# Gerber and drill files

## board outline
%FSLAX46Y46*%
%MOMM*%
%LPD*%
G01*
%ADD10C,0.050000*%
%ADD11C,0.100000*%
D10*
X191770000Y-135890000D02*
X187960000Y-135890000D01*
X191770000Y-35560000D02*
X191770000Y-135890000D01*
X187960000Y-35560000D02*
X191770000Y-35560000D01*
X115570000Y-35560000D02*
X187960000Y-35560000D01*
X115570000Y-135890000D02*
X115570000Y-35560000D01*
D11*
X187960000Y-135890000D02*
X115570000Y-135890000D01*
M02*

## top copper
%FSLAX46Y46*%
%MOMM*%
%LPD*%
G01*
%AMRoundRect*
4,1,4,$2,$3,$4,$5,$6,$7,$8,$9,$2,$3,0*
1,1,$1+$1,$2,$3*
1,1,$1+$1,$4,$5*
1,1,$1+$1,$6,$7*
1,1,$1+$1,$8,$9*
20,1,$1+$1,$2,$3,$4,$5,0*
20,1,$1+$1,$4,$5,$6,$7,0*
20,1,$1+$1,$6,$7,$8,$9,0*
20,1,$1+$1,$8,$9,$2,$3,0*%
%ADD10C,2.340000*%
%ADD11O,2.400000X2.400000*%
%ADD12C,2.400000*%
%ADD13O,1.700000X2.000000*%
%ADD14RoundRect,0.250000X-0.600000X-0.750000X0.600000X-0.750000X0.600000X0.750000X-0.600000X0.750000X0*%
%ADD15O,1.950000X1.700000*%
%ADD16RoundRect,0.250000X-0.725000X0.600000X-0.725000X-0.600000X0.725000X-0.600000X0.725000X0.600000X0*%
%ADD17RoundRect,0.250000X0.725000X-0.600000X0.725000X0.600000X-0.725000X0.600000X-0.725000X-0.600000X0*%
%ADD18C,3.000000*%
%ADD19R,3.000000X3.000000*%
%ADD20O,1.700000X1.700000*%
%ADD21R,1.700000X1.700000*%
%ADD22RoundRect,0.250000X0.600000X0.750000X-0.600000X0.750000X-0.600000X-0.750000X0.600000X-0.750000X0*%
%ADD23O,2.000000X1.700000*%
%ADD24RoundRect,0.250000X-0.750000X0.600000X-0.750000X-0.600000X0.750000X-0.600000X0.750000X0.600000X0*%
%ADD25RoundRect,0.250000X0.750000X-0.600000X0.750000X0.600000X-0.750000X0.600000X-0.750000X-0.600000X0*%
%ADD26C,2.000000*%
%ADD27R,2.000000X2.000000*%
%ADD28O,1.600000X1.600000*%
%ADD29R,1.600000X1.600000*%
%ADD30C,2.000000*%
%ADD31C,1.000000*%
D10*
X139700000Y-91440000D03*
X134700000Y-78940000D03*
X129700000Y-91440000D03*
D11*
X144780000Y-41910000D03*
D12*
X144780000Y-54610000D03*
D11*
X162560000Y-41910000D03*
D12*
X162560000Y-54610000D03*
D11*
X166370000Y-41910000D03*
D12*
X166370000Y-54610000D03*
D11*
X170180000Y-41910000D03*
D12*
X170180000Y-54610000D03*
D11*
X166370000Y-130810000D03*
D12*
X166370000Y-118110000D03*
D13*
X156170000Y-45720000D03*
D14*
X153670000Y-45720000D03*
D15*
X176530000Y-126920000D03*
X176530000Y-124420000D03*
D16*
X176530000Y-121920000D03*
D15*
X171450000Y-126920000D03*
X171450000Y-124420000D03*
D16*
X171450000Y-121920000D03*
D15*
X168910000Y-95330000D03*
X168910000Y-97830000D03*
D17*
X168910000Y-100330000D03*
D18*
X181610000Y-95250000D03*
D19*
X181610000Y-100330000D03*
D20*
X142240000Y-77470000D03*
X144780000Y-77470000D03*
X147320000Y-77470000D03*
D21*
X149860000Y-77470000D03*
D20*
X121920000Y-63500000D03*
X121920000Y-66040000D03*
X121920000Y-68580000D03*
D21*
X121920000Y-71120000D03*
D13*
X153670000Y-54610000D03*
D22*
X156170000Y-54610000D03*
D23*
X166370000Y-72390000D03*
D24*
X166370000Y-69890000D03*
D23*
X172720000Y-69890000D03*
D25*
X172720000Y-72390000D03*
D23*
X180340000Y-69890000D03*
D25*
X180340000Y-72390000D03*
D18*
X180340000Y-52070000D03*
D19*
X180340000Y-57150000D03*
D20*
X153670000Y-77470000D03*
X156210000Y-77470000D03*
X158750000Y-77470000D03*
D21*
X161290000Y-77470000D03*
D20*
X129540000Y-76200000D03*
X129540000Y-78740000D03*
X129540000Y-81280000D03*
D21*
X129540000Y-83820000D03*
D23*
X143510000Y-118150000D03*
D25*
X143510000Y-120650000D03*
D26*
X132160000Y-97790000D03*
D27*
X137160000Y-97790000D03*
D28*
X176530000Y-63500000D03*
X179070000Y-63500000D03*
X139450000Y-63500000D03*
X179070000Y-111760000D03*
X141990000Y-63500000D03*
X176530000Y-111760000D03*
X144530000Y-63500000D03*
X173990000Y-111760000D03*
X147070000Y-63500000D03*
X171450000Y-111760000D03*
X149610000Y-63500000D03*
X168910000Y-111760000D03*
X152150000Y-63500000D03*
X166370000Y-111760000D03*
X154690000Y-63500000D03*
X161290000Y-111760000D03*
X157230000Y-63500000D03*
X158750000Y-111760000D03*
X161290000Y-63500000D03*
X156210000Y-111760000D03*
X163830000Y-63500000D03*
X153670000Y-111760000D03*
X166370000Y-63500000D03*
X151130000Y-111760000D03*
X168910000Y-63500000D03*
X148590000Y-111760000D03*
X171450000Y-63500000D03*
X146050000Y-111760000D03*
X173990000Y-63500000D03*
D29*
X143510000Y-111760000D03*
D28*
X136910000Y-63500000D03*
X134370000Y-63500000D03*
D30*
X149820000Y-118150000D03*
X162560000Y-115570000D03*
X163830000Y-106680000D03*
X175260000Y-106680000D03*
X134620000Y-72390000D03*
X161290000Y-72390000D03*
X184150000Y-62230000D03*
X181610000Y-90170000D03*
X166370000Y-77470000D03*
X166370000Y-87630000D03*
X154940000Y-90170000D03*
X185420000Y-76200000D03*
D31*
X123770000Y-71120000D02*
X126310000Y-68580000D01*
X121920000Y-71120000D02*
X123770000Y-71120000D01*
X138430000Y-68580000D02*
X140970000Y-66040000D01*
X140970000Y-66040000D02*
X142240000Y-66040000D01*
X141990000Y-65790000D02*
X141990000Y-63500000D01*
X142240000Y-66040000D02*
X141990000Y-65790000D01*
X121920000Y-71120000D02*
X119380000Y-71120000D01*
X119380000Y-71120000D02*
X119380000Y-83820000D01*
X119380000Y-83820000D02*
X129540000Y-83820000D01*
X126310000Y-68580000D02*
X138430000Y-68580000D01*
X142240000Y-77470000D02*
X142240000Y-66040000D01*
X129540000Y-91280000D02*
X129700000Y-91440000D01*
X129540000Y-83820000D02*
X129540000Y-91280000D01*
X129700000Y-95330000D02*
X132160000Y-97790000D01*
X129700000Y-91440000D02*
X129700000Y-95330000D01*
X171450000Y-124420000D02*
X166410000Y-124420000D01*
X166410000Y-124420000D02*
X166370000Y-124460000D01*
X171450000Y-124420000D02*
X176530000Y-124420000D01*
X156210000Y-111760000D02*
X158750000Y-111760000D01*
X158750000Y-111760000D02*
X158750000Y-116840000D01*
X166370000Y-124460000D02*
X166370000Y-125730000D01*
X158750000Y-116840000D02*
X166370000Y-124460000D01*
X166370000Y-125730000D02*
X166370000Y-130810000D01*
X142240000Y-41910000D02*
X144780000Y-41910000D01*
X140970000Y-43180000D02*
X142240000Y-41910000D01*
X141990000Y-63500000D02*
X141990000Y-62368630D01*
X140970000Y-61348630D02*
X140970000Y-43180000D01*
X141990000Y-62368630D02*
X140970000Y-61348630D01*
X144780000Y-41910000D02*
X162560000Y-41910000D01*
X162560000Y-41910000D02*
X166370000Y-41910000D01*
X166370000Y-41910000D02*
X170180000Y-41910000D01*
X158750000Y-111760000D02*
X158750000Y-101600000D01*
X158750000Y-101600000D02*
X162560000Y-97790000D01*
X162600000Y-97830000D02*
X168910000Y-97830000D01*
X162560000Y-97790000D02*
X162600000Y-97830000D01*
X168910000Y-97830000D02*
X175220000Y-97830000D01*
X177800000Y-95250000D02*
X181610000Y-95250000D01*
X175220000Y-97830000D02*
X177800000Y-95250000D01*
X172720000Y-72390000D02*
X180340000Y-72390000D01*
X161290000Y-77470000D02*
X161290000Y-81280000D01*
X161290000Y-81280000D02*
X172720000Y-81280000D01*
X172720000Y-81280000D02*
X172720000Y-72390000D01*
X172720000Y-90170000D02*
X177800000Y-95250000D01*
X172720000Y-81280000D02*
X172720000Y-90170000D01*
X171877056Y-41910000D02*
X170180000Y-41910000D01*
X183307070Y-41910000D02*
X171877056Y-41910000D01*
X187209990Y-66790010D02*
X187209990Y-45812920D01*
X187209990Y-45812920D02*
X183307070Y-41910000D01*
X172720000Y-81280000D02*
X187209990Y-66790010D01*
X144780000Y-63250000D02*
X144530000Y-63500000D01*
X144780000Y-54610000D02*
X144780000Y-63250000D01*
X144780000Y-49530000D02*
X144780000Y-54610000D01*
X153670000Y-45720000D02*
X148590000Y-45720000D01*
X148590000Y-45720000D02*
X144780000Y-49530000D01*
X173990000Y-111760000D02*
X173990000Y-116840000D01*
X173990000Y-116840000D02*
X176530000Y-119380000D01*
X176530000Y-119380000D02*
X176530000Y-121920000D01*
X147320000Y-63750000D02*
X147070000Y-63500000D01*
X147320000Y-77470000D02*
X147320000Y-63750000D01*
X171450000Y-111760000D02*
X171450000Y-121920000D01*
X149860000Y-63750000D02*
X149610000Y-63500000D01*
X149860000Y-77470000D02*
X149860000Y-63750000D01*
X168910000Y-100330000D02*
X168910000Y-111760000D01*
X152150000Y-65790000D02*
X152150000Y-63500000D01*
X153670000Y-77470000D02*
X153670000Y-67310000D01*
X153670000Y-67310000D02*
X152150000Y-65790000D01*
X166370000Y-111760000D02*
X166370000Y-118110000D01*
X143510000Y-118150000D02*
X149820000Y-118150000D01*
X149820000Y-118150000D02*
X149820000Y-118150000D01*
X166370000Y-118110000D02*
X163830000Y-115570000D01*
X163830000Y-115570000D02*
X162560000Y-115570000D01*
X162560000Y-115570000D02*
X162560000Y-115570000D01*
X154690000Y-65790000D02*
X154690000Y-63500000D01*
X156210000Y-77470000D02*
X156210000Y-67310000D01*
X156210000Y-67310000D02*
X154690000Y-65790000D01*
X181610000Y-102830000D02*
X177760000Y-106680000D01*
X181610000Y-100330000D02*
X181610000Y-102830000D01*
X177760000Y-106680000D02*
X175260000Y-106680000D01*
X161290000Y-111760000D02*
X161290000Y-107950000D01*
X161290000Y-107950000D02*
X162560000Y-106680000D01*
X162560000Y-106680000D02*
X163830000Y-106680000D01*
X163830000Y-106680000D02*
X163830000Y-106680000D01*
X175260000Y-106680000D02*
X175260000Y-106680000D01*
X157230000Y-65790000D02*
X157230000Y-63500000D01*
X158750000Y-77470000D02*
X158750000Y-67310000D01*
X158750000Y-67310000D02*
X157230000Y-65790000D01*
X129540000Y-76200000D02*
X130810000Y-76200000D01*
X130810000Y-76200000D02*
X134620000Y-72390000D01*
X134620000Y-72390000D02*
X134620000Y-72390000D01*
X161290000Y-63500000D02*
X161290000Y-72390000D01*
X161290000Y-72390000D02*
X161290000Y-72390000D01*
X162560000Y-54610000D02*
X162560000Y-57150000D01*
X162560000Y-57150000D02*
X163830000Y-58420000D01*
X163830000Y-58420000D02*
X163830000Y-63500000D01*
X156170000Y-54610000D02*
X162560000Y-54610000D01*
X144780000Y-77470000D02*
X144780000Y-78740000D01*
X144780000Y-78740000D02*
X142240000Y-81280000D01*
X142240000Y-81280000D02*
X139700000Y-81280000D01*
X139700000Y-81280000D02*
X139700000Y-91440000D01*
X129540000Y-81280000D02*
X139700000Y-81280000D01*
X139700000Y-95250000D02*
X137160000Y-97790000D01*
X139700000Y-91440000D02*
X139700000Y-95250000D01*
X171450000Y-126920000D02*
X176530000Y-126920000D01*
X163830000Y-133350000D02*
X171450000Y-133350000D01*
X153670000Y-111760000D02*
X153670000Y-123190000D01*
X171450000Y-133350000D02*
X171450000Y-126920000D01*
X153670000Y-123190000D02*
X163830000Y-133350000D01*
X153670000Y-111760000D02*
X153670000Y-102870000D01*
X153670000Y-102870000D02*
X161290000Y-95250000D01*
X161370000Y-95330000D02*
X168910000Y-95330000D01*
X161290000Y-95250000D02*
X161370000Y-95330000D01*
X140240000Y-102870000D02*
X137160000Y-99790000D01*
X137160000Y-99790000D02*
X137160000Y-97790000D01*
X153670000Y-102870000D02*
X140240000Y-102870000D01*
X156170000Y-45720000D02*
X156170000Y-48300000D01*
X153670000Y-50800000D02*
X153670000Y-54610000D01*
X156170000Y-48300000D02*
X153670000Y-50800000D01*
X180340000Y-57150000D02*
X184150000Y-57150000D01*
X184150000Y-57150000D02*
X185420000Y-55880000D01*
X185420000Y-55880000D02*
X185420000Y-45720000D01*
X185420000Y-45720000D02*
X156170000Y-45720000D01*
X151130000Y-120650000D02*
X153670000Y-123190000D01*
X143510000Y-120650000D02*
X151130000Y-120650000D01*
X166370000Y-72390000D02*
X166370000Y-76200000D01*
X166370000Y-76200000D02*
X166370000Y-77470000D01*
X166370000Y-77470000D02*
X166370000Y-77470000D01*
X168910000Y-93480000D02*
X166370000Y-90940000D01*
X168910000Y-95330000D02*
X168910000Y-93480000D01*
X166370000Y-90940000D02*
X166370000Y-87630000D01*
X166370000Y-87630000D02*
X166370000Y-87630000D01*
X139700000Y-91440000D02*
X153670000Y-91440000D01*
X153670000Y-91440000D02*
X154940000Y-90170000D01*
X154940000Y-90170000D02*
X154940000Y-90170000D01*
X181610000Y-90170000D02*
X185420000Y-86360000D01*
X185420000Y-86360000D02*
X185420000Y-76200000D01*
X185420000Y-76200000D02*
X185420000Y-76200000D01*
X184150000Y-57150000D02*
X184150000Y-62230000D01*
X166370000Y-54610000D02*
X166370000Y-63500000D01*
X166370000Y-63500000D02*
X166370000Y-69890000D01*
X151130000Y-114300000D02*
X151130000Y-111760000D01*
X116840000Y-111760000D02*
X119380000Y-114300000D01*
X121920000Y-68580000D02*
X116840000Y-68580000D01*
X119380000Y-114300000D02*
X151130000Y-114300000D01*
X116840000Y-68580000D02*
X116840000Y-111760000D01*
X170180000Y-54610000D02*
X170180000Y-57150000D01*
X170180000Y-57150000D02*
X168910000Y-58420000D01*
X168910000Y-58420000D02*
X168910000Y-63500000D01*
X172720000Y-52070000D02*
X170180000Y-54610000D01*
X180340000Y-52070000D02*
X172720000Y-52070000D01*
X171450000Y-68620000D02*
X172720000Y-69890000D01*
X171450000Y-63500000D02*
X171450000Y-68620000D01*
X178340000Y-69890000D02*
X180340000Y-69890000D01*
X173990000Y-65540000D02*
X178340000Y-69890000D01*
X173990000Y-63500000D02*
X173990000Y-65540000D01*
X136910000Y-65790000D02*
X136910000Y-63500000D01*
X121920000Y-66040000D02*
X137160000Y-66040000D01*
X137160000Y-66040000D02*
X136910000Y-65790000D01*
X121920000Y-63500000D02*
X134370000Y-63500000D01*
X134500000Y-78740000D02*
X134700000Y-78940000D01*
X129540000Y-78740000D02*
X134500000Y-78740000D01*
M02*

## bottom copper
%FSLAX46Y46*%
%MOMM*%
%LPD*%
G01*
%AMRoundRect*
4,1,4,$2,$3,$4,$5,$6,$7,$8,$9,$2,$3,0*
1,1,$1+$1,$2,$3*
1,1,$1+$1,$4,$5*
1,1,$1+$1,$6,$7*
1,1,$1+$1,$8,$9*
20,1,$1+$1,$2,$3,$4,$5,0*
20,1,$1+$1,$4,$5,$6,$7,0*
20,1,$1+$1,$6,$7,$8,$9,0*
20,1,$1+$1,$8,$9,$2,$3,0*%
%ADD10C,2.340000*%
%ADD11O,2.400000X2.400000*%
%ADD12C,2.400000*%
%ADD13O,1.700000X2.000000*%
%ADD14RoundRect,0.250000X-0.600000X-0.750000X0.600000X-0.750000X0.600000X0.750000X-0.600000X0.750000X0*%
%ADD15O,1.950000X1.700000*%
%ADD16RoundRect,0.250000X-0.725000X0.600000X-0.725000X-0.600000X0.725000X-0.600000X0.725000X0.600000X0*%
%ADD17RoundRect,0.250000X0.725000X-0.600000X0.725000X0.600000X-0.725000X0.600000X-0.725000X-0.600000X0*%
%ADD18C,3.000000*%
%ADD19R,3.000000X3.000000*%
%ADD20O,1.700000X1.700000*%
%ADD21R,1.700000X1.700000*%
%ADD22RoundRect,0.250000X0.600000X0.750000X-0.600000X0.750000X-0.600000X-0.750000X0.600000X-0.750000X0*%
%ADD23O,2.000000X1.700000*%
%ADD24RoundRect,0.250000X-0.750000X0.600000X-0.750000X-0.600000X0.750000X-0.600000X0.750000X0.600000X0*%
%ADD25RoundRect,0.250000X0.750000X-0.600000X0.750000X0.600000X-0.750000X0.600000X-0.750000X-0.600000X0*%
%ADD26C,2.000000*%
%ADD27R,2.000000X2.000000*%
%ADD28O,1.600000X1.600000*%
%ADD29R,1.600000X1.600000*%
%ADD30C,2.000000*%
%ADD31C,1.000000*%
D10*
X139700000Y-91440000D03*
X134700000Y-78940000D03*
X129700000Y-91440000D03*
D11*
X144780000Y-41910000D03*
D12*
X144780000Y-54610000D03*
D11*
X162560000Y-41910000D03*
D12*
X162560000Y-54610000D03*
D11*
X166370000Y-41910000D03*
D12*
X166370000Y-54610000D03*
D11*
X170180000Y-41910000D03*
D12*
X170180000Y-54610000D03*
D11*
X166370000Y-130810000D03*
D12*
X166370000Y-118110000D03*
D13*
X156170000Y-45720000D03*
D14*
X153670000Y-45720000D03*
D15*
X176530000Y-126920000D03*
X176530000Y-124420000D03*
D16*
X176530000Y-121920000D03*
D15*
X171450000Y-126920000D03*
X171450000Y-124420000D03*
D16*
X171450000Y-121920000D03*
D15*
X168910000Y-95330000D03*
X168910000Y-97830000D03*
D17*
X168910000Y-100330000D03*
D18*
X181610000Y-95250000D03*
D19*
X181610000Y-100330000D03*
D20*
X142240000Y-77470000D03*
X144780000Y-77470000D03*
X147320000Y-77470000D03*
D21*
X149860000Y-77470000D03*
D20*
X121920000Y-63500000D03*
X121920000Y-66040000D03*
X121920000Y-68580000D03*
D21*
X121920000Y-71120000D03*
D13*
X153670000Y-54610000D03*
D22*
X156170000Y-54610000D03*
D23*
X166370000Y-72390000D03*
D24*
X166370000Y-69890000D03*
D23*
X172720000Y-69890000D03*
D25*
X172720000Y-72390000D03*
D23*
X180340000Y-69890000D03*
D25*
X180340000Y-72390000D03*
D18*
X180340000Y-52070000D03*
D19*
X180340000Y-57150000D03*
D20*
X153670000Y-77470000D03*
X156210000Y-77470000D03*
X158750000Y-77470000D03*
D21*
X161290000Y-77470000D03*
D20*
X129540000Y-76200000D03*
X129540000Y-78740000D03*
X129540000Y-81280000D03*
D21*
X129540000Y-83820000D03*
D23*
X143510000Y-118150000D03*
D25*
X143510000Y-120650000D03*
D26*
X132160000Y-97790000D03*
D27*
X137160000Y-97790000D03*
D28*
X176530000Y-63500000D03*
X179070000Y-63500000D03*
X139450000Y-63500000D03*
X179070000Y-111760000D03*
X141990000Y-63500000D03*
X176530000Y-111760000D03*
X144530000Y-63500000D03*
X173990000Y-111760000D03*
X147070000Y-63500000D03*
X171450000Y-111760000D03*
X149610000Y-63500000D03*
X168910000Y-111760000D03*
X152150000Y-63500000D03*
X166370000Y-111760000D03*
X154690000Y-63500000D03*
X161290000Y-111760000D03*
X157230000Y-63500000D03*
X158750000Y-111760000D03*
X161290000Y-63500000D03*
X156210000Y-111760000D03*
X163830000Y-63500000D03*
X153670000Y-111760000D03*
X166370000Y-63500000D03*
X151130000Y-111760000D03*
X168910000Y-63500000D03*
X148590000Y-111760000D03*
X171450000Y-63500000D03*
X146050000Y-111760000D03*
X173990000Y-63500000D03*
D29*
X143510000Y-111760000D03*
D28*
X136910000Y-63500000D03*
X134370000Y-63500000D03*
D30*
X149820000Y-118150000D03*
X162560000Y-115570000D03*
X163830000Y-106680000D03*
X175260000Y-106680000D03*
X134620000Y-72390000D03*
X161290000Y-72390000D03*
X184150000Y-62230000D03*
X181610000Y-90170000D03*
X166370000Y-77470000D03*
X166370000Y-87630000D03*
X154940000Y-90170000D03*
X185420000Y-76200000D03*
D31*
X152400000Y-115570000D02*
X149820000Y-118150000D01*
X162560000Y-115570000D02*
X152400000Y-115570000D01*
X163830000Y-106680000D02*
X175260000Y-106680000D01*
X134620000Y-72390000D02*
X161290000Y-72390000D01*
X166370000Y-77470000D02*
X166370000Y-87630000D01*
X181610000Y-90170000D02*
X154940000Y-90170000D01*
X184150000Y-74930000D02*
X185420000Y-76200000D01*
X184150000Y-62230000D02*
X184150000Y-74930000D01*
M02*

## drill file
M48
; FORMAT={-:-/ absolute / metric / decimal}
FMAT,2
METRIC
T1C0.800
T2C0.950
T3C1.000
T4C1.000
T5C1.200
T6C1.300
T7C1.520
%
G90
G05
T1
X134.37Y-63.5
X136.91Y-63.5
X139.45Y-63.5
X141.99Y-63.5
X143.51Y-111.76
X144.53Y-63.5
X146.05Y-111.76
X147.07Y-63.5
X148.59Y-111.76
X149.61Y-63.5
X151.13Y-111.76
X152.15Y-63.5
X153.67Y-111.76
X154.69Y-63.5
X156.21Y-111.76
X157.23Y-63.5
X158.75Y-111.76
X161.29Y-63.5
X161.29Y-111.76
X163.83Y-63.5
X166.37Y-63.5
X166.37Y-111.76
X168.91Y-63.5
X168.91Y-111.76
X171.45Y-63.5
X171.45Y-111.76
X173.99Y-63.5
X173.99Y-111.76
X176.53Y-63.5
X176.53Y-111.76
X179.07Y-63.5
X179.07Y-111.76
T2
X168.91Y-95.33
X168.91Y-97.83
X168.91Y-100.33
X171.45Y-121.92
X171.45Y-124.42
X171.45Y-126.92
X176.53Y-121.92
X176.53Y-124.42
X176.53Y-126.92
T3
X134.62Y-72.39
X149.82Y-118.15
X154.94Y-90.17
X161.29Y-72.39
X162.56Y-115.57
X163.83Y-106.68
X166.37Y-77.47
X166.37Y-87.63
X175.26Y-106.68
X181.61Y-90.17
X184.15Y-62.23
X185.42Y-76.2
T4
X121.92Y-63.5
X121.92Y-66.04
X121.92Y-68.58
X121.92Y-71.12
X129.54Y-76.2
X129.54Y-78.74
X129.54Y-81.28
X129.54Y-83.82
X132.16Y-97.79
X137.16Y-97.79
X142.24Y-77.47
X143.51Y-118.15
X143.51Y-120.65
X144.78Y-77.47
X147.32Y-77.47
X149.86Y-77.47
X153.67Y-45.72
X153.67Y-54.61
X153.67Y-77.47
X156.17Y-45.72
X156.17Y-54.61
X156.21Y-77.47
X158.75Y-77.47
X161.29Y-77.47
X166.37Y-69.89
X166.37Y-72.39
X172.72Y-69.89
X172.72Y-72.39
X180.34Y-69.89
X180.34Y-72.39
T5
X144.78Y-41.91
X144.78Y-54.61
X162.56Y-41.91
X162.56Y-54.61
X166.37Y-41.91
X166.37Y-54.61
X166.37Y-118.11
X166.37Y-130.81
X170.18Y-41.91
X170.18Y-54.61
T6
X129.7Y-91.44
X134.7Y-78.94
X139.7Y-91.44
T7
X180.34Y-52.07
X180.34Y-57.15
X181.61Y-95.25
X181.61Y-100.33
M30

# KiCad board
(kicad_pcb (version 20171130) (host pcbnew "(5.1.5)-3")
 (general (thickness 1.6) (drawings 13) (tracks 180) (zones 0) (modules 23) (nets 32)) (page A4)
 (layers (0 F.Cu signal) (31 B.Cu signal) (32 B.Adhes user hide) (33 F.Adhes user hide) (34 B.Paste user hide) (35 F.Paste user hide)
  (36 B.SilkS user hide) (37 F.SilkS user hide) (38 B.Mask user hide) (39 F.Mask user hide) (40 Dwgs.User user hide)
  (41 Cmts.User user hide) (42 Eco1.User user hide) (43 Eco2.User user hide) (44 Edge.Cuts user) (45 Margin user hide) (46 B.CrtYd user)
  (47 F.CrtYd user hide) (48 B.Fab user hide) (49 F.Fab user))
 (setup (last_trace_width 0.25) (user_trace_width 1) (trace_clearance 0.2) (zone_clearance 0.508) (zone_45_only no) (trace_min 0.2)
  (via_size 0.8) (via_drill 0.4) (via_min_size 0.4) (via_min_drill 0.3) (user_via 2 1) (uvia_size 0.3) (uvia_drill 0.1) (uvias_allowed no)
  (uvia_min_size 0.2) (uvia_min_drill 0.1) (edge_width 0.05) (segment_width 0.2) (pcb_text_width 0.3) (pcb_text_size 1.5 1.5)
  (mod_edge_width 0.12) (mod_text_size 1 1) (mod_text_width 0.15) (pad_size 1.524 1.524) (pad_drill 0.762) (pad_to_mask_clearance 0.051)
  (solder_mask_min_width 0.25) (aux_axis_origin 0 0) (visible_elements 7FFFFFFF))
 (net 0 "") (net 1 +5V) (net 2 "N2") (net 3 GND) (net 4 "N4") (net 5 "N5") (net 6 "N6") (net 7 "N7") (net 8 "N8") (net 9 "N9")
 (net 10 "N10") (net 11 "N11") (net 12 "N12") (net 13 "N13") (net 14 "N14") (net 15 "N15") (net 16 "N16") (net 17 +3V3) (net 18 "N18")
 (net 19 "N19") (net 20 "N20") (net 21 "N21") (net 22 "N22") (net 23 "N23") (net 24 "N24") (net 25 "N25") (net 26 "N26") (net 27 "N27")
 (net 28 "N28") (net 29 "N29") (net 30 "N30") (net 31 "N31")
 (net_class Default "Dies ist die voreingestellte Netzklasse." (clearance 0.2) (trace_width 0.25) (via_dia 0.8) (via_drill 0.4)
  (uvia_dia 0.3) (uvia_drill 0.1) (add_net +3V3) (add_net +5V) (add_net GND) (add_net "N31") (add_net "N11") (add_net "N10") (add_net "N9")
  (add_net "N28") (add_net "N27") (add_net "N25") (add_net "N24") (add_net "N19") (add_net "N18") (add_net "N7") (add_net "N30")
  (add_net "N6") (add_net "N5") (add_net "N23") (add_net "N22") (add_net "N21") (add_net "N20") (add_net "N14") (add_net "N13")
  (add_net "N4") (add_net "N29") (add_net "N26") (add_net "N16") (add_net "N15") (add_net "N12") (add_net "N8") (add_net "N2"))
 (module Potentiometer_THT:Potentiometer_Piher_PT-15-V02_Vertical (layer F.Cu) (at 139.7 91.44 90)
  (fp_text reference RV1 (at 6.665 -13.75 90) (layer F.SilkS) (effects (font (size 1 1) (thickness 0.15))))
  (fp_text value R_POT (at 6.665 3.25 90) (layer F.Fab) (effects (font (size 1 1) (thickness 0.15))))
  (pad 1 thru_hole circle (at 0 0 90) (size 2.34 2.34) (drill 1.3) (layers *.Cu *.Mask) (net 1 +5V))
  (pad 2 thru_hole circle (at 12.5 -5 90) (size 2.34 2.34) (drill 1.3) (layers *.Cu *.Mask) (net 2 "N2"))
  (pad 3 thru_hole circle (at 0 -10 90) (size 2.34 2.34) (drill 1.3) (layers *.Cu *.Mask) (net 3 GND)))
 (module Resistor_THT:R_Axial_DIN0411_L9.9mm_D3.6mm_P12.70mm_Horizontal (layer F.Cu) (at 144.78 54.61 90)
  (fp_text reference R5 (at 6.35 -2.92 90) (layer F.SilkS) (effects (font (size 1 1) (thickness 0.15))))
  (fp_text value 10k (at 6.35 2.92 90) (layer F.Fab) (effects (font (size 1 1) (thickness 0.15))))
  (pad 2 thru_hole oval (at 12.7 0 90) (size 2.4 2.4) (drill 1.2) (layers *.Cu *.Mask) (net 3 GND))
  (pad 1 thru_hole circle (at 0 0 90) (size 2.4 2.4) (drill 1.2) (layers *.Cu *.Mask) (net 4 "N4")))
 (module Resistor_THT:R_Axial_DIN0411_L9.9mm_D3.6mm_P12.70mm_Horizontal (layer F.Cu) (at 162.56 54.61 90)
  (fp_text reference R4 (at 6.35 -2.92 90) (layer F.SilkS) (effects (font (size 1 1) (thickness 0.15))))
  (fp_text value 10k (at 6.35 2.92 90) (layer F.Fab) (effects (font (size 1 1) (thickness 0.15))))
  (pad 2 thru_hole oval (at 12.7 0 90) (size 2.4 2.4) (drill 1.2) (layers *.Cu *.Mask) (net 3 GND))
  (pad 1 thru_hole circle (at 0 0 90) (size 2.4 2.4) (drill 1.2) (layers *.Cu *.Mask) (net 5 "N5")))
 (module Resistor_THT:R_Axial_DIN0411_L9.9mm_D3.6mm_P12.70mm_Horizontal (layer F.Cu) (at 166.37 54.61 90)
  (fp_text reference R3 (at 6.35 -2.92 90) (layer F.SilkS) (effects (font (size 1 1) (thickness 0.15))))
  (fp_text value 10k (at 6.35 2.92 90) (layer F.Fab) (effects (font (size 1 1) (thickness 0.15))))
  (pad 2 thru_hole oval (at 12.7 0 90) (size 2.4 2.4) (drill 1.2) (layers *.Cu *.Mask) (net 3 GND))
  (pad 1 thru_hole circle (at 0 0 90) (size 2.4 2.4) (drill 1.2) (layers *.Cu *.Mask) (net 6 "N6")))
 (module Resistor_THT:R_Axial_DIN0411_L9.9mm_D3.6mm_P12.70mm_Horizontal (layer F.Cu) (at 170.18 54.61 90)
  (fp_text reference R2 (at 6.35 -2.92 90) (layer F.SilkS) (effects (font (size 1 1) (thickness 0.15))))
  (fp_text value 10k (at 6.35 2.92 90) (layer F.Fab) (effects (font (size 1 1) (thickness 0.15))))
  (pad 2 thru_hole oval (at 12.7 0 90) (size 2.4 2.4) (drill 1.2) (layers *.Cu *.Mask) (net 3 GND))
  (pad 1 thru_hole circle (at 0 0 90) (size 2.4 2.4) (drill 1.2) (layers *.Cu *.Mask) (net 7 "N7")))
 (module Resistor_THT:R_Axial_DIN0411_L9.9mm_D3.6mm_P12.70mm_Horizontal (layer F.Cu) (at 166.37 118.11 270)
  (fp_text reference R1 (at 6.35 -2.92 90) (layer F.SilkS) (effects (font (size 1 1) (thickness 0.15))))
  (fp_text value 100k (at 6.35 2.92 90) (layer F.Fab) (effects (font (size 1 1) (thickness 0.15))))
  (pad 2 thru_hole oval (at 12.7 0 270) (size 2.4 2.4) (drill 1.2) (layers *.Cu *.Mask) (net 3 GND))
  (pad 1 thru_hole circle (at 0 0 270) (size 2.4 2.4) (drill 1.2) (layers *.Cu *.Mask) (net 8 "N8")))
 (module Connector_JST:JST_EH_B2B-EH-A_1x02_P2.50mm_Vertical (layer F.Cu) (at 153.67 45.72)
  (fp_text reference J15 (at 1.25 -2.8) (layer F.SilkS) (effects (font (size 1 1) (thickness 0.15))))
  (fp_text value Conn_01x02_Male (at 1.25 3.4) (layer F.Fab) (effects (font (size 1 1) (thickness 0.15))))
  (pad 2 thru_hole oval (at 2.5 0) (size 1.7 2) (drill 1) (layers *.Cu *.Mask) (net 1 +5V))
  (pad 1 thru_hole roundrect (at 0 0) (size 1.7 2) (drill 1) (layers *.Cu *.Mask) (roundrect_rratio 0.147059) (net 4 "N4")))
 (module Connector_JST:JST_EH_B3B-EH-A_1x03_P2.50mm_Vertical (layer F.Cu) (at 176.53 121.92 270)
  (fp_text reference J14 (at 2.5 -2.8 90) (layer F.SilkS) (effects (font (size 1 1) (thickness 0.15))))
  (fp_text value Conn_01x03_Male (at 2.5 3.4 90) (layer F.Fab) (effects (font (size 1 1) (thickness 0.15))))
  (pad 3 thru_hole oval (at 5 0 270) (size 1.7 1.95) (drill 0.95) (layers *.Cu *.Mask) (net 1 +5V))
  (pad 2 thru_hole oval (at 2.5 0 270) (size 1.7 1.95) (drill 0.95) (layers *.Cu *.Mask) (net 3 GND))
  (pad 1 thru_hole roundrect (at 0 0 270) (size 1.7 1.95) (drill 0.95) (layers *.Cu *.Mask) (roundrect_rratio 0.147059) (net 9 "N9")))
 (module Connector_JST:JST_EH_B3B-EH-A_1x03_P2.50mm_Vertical (layer F.Cu) (at 171.45 121.92 270)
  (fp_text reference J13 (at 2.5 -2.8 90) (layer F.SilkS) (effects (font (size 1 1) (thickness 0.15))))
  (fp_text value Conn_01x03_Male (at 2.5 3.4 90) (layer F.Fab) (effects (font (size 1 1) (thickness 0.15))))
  (pad 3 thru_hole oval (at 5 0 270) (size 1.7 1.95) (drill 0.95) (layers *.Cu *.Mask) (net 1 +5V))
  (pad 2 thru_hole oval (at 2.5 0 270) (size 1.7 1.95) (drill 0.95) (layers *.Cu *.Mask) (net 3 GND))
  (pad 1 thru_hole roundrect (at 0 0 270) (size 1.7 1.95) (drill 0.95) (layers *.Cu *.Mask) (roundrect_rratio 0.147059) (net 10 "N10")))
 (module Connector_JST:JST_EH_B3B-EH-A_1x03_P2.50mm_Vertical (layer F.Cu) (at 168.91 100.33 90)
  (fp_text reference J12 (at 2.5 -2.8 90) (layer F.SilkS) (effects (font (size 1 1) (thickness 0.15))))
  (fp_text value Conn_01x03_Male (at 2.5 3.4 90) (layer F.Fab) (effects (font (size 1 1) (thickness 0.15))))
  (pad 3 thru_hole oval (at 5 0 90) (size 1.7 1.95) (drill 0.95) (layers *.Cu *.Mask) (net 1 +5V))
  (pad 2 thru_hole oval (at 2.5 0 90) (size 1.7 1.95) (drill 0.95) (layers *.Cu *.Mask) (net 3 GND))
  (pad 1 thru_hole roundrect (at 0 0 90) (size 1.7 1.95) (drill 0.95) (layers *.Cu *.Mask) (roundrect_rratio 0.147059) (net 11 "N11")))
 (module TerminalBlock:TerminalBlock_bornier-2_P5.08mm (layer F.Cu) (at 181.61 100.33 90)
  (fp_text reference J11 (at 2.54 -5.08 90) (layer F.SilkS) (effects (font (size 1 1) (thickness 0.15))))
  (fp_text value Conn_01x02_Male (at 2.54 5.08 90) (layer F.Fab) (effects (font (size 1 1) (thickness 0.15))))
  (pad 2 thru_hole circle (at 5.08 0 90) (size 3 3) (drill 1.52) (layers *.Cu *.Mask) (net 3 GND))
  (pad 1 thru_hole rect (at 0 0 90) (size 3 3) (drill 1.52) (layers *.Cu *.Mask) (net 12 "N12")))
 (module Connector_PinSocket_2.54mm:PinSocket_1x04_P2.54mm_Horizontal (layer F.Cu) (at 149.86 77.47 270)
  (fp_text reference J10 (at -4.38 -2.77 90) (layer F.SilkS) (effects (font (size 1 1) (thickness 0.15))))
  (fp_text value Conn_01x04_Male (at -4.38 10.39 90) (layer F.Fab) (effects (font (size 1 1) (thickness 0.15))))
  (pad 4 thru_hole oval (at 0 7.62 270) (size 1.7 1.7) (drill 1) (layers *.Cu *.Mask) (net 3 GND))
  (pad 3 thru_hole oval (at 0 5.08 270) (size 1.7 1.7) (drill 1) (layers *.Cu *.Mask) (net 1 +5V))
  (pad 2 thru_hole oval (at 0 2.54 270) (size 1.7 1.7) (drill 1) (layers *.Cu *.Mask) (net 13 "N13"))
  (pad 1 thru_hole rect (at 0 0 270) (size 1.7 1.7) (drill 1) (layers *.Cu *.Mask) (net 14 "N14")))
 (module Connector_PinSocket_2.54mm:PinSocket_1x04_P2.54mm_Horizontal (layer F.Cu) (at 121.92 71.12 180)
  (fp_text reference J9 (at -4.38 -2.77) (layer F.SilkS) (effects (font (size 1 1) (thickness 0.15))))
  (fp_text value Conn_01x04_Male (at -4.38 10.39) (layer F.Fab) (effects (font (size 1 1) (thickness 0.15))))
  (pad 4 thru_hole oval (at 0 7.62 180) (size 1.7 1.7) (drill 1) (layers *.Cu *.Mask) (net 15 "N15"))
  (pad 3 thru_hole oval (at 0 5.08 180) (size 1.7 1.7) (drill 1) (layers *.Cu *.Mask) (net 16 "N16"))
  (pad 2 thru_hole oval (at 0 2.54 180) (size 1.7 1.7) (drill 1) (layers *.Cu *.Mask) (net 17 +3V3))
  (pad 1 thru_hole rect (at 0 0 180) (size 1.7 1.7) (drill 1) (layers *.Cu *.Mask) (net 3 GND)))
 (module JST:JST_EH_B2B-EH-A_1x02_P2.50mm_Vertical (layer F.Cu) (at 156.17 54.61 180)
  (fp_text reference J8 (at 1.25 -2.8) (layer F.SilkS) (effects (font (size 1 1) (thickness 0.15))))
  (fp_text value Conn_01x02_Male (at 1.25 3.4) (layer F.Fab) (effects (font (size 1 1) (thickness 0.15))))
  (pad 2 thru_hole oval (at 2.5 0 180) (size 1.7 2) (drill 1) (layers *.Cu *.Mask) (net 1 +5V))
  (pad 1 thru_hole roundrect (at 0 0 180) (size 1.7 2) (drill 1) (layers *.Cu *.Mask) (roundrect_rratio 0.147059) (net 5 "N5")))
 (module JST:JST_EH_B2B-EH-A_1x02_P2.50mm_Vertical (layer F.Cu) (at 166.37 69.89 270)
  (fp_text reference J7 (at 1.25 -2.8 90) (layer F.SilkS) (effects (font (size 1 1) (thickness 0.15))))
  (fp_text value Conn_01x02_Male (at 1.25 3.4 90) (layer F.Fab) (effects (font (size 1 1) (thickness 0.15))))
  (pad 2 thru_hole oval (at 2.5 0 270) (size 1.7 2) (drill 1) (layers *.Cu *.Mask) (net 1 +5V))
  (pad 1 thru_hole roundrect (at 0 0 270) (size 1.7 2) (drill 1) (layers *.Cu *.Mask) (roundrect_rratio 0.147059) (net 6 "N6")))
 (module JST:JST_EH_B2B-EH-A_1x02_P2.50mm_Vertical (layer F.Cu) (at 172.72 72.39 90)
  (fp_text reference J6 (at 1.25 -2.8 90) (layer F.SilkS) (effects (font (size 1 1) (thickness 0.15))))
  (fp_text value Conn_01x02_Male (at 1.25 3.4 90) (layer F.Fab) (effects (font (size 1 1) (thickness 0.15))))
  (pad 2 thru_hole oval (at 2.5 0 90) (size 1.7 2) (drill 1) (layers *.Cu *.Mask) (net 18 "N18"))
  (pad 1 thru_hole roundrect (at 0 0 90) (size 1.7 2) (drill 1) (layers *.Cu *.Mask) (roundrect_rratio 0.147059) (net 3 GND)))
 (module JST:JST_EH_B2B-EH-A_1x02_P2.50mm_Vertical (layer F.Cu) (at 180.34 72.39 90)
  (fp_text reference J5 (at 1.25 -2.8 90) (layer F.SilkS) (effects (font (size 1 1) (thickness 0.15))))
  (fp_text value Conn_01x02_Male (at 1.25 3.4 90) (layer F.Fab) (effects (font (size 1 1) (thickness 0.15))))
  (pad 2 thru_hole oval (at 2.5 0 90) (size 1.7 2) (drill 1) (layers *.Cu *.Mask) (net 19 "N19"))
  (pad 1 thru_hole roundrect (at 0 0 90) (size 1.7 2) (drill 1) (layers *.Cu *.Mask) (roundrect_rratio 0.147059) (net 3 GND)))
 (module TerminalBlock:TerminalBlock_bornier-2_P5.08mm (layer F.Cu) (at 180.34 57.15 90)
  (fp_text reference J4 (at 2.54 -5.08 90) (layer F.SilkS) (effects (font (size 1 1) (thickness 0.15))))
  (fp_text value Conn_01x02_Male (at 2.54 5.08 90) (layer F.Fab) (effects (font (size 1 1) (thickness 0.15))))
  (pad 2 thru_hole circle (at 5.08 0 90) (size 3 3) (drill 1.52) (layers *.Cu *.Mask) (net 7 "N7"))
  (pad 1 thru_hole rect (at 0 0 90) (size 3 3) (drill 1.52) (layers *.Cu *.Mask) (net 1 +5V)))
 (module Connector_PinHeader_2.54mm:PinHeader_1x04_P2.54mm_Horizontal (layer F.Cu) (at 161.29 77.47 270)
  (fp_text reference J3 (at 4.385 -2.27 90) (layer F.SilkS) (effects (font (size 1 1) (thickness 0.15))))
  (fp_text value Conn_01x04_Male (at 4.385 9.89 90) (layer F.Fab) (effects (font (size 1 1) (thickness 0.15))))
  (pad 4 thru_hole oval (at 0 7.62 270) (size 1.7 1.7) (drill 1) (layers *.Cu *.Mask) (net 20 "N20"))
  (pad 3 thru_hole oval (at 0 5.08 270) (size 1.7 1.7) (drill 1) (layers *.Cu *.Mask) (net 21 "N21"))
  (pad 2 thru_hole oval (at 0 2.54 270) (size 1.7 1.7) (drill 1) (layers *.Cu *.Mask) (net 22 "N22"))
  (pad 1 thru_hole rect (at 0 0 270) (size 1.7 1.7) (drill 1) (layers *.Cu *.Mask) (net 3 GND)))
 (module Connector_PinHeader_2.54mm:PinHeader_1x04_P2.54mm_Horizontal (layer F.Cu) (at 129.54 83.82 180)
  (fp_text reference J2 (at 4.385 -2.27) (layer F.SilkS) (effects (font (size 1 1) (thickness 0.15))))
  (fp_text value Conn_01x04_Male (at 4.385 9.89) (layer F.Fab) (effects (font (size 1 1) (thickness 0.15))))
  (pad 4 thru_hole oval (at 0 7.62 180) (size 1.7 1.7) (drill 1) (layers *.Cu *.Mask) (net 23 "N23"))
  (pad 3 thru_hole oval (at 0 5.08 180) (size 1.7 1.7) (drill 1) (layers *.Cu *.Mask) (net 2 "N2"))
  (pad 2 thru_hole oval (at 0 2.54 180) (size 1.7 1.7) (drill 1) (layers *.Cu *.Mask) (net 1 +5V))
  (pad 1 thru_hole rect (at 0 0 180) (size 1.7 1.7) (drill 1) (layers *.Cu *.Mask) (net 3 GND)))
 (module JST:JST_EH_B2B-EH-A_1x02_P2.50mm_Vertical (layer F.Cu) (at 143.51 120.65 90)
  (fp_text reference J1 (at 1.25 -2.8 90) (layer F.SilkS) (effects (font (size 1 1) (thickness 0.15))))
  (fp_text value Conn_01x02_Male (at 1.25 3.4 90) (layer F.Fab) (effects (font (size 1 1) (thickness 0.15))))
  (pad 2 thru_hole oval (at 2.5 0 90) (size 1.7 2) (drill 1) (layers *.Cu *.Mask) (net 8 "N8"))
  (pad 1 thru_hole roundrect (at 0 0 90) (size 1.7 2) (drill 1) (layers *.Cu *.Mask) (roundrect_rratio 0.147059) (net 1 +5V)))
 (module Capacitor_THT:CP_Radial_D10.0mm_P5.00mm (layer F.Cu) (at 137.16 97.79 180)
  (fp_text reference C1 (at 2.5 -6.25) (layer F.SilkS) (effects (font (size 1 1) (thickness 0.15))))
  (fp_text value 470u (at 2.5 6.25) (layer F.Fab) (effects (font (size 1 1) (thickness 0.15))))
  (pad 2 thru_hole circle (at 5 0 180) (size 2 2) (drill 1) (layers *.Cu *.Mask) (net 3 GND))
  (pad 1 thru_hole rect (at 0 0 180) (size 2 2) (drill 1) (layers *.Cu *.Mask) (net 1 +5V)))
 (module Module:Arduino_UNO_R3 (layer B.Cu) (at 143.51 111.76)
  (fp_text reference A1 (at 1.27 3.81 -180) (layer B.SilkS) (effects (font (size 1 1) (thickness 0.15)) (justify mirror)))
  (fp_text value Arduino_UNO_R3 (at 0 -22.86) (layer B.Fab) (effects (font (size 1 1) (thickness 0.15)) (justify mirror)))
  (pad 16 thru_hole oval (at 33.02 -48.26 270) (size 1.6 1.6) (drill 0.8) (layers *.Cu *.Mask) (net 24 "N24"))
  (pad 15 thru_hole oval (at 35.56 -48.26 270) (size 1.6 1.6) (drill 0.8) (layers *.Cu *.Mask) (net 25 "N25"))
  (pad 30 thru_hole oval (at -4.06 -48.26 270) (size 1.6 1.6) (drill 0.8) (layers *.Cu *.Mask) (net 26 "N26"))
  (pad 14 thru_hole oval (at 35.56 0 270) (size 1.6 1.6) (drill 0.8) (layers *.Cu *.Mask) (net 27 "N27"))
  (pad 29 thru_hole oval (at -1.52 -48.26 270) (size 1.6 1.6) (drill 0.8) (layers *.Cu *.Mask) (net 3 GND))
  (pad 13 thru_hole oval (at 33.02 0 270) (size 1.6 1.6) (drill 0.8) (layers *.Cu *.Mask) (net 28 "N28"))
  (pad 28 thru_hole oval (at 1.02 -48.26 270) (size 1.6 1.6) (drill 0.8) (layers *.Cu *.Mask) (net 4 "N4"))
  (pad 12 thru_hole oval (at 30.48 0 270) (size 1.6 1.6) (drill 0.8) (layers *.Cu *.Mask) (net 9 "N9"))
  (pad 27 thru_hole oval (at 3.56 -48.26 270) (size 1.6 1.6) (drill 0.8) (layers *.Cu *.Mask) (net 13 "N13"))
  (pad 11 thru_hole oval (at 27.94 0 270) (size 1.6 1.6) (drill 0.8) (layers *.Cu *.Mask) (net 10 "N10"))
  (pad 26 thru_hole oval (at 6.1 -48.26 270) (size 1.6 1.6) (drill 0.8) (layers *.Cu *.Mask) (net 14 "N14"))
  (pad 10 thru_hole oval (at 25.4 0 270) (size 1.6 1.6) (drill 0.8) (layers *.Cu *.Mask) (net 11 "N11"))
  (pad 25 thru_hole oval (at 8.64 -48.26 270) (size 1.6 1.6) (drill 0.8) (layers *.Cu *.Mask) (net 20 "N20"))
  (pad 9 thru_hole oval (at 22.86 0 270) (size 1.6 1.6) (drill 0.8) (layers *.Cu *.Mask) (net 8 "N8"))
  (pad 24 thru_hole oval (at 11.18 -48.26 270) (size 1.6 1.6) (drill 0.8) (layers *.Cu *.Mask) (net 21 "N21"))
  (pad 8 thru_hole oval (at 17.78 0 270) (size 1.6 1.6) (drill 0.8) (layers *.Cu *.Mask) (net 12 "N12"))
  (pad 23 thru_hole oval (at 13.72 -48.26 270) (size 1.6 1.6) (drill 0.8) (layers *.Cu *.Mask) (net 22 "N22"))
  (pad 7 thru_hole oval (at 15.24 0 270) (size 1.6 1.6) (drill 0.8) (layers *.Cu *.Mask) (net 3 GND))
  (pad 22 thru_hole oval (at 17.78 -48.26 270) (size 1.6 1.6) (drill 0.8) (layers *.Cu *.Mask) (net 23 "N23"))
  (pad 6 thru_hole oval (at 12.7 0 270) (size 1.6 1.6) (drill 0.8) (layers *.Cu *.Mask) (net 3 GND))
  (pad 21 thru_hole oval (at 20.32 -48.26 270) (size 1.6 1.6) (drill 0.8) (layers *.Cu *.Mask) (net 5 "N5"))
  (pad 5 thru_hole oval (at 10.16 0 270) (size 1.6 1.6) (drill 0.8) (layers *.Cu *.Mask) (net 1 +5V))
  (pad 20 thru_hole oval (at 22.86 -48.26 270) (size 1.6 1.6) (drill 0.8) (layers *.Cu *.Mask) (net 6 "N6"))
  (pad 4 thru_hole oval (at 7.62 0 270) (size 1.6 1.6) (drill 0.8) (layers *.Cu *.Mask) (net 17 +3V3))
  (pad 19 thru_hole oval (at 25.4 -48.26 270) (size 1.6 1.6) (drill 0.8) (layers *.Cu *.Mask) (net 7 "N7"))
  (pad 3 thru_hole oval (at 5.08 0 270) (size 1.6 1.6) (drill 0.8) (layers *.Cu *.Mask) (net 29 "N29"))
  (pad 18 thru_hole oval (at 27.94 -48.26 270) (size 1.6 1.6) (drill 0.8) (layers *.Cu *.Mask) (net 18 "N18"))
  (pad 2 thru_hole oval (at 2.54 0 270) (size 1.6 1.6) (drill 0.8) (layers *.Cu *.Mask) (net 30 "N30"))
  (pad 17 thru_hole oval (at 30.48 -48.26 270) (size 1.6 1.6) (drill 0.8) (layers *.Cu *.Mask) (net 19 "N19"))
  (pad 1 thru_hole rect (at 0 0 270) (size 1.6 1.6) (drill 0.8) (layers *.Cu *.Mask) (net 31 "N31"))
  (pad 31 thru_hole oval (at -6.6 -48.26 270) (size 1.6 1.6) (drill 0.8) (layers *.Cu *.Mask) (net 16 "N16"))
  (pad 32 thru_hole oval (at -9.14 -48.26 270) (size 1.6 1.6) (drill 0.8) (layers *.Cu *.Mask) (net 15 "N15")))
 (gr_line (start 191.77 135.89) (end 187.96 135.89) (layer Edge.Cuts) (width 0.05))
 (gr_line (start 191.77 35.56) (end 191.77 135.89) (layer Edge.Cuts) (width 0.05))
 (gr_line (start 187.96 35.56) (end 191.77 35.56) (layer Edge.Cuts) (width 0.05))
 (gr_line (start 115.57 35.56) (end 187.96 35.56) (layer Edge.Cuts) (width 0.05))
 (gr_line (start 115.57 135.89) (end 115.57 35.56) (layer Edge.Cuts) (width 0.05))
 (gr_line (start 187.96 135.89) (end 115.57 135.89) (layer Edge.Cuts) (width 0.1))
 (segment (start 123.77 71.12) (end 126.31 68.58) (width 1) (layer F.Cu) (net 3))
 (segment (start 121.92 71.12) (end 123.77 71.12) (width 1) (layer F.Cu) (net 3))
 (segment (start 138.43 68.58) (end 140.97 66.04) (width 1) (layer F.Cu) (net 3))
 (segment (start 140.97 66.04) (end 142.24 66.04) (width 1) (layer F.Cu) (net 3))
 (segment (start 141.99 65.79) (end 141.99 63.5) (width 1) (layer F.Cu) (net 3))
 (segment (start 142.24 66.04) (end 141.99 65.79) (width 1) (layer F.Cu) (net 3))
 (segment (start 121.92 71.12) (end 119.38 71.12) (width 1) (layer F.Cu) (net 3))
 (segment (start 119.38 71.12) (end 119.38 83.82) (width 1) (layer F.Cu) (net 3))
 (segment (start 119.38 83.82) (end 129.54 83.82) (width 1) (layer F.Cu) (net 3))
 (segment (start 126.31 68.58) (end 138.43 68.58) (width 1) (layer F.Cu) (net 3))
 (segment (start 142.24 77.47) (end 142.24 66.04) (width 1) (layer F.Cu) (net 3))
 (segment (start 129.54 91.28) (end 129.7 91.44) (width 1) (layer F.Cu) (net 3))
 (segment (start 129.54 83.82) (end 129.54 91.28) (width 1) (layer F.Cu) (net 3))
 (segment (start 129.7 95.33) (end 132.16 97.79) (width 1) (layer F.Cu) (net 3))
 (segment (start 129.7 91.44) (end 129.7 95.33) (width 1) (layer F.Cu) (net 3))
 (segment (start 171.45 124.42) (end 166.41 124.42) (width 1) (layer F.Cu) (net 3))
 (segment (start 166.41 124.42) (end 166.37 124.46) (width 1) (layer F.Cu) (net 3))
 (segment (start 171.45 124.42) (end 176.53 124.42) (width 1) (layer F.Cu) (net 3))
 (segment (start 156.21 111.76) (end 158.75 111.76) (width 1) (layer F.Cu) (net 3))
 (segment (start 158.75 111.76) (end 158.75 116.84) (width 1) (layer F.Cu) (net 3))
 (segment (start 166.37 124.46) (end 166.37 125.73) (width 1) (layer F.Cu) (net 3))
 (segment (start 158.75 116.84) (end 166.37 124.46) (width 1) (layer F.Cu) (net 3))
 (segment (start 166.37 125.73) (end 166.37 130.81) (width 1) (layer F.Cu) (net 3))
 (segment (start 142.24 41.91) (end 144.78 41.91) (width 1) (layer F.Cu) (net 3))
 (segment (start 140.97 43.18) (end 142.24 41.91) (width 1) (layer F.Cu) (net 3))
 (segment (start 141.99 63.5) (end 141.99 62.36863) (width 1) (layer F.Cu) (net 3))
 (segment (start 140.97 61.34863) (end 140.97 43.18) (width 1) (layer F.Cu) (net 3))
 (segment (start 141.99 62.36863) (end 140.97 61.34863) (width 1) (layer F.Cu) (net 3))
 (segment (start 144.78 41.91) (end 162.56 41.91) (width 1) (layer F.Cu) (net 3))
 (segment (start 162.56 41.91) (end 166.37 41.91) (width 1) (layer F.Cu) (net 3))
 (segment (start 166.37 41.91) (end 170.18 41.91) (width 1) (layer F.Cu) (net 3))
 (segment (start 158.75 111.76) (end 158.75 101.6) (width 1) (layer F.Cu) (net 3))
 (segment (start 158.75 101.6) (end 162.56 97.79) (width 1) (layer F.Cu) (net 3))
 (segment (start 162.6 97.83) (end 168.91 97.83) (width 1) (layer F.Cu) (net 3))
 (segment (start 162.56 97.79) (end 162.6 97.83) (width 1) (layer F.Cu) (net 3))
 (segment (start 168.91 97.83) (end 175.22 97.83) (width 1) (layer F.Cu) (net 3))
 (segment (start 177.8 95.25) (end 181.61 95.25) (width 1) (layer F.Cu) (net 3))
 (segment (start 175.22 97.83) (end 177.8 95.25) (width 1) (layer F.Cu) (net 3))
 (segment (start 172.72 72.39) (end 180.34 72.39) (width 1) (layer F.Cu) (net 3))
 (segment (start 161.29 77.47) (end 161.29 81.28) (width 1) (layer F.Cu) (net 3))
 (segment (start 161.29 81.28) (end 172.72 81.28) (width 1) (layer F.Cu) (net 3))
 (segment (start 172.72 81.28) (end 172.72 72.39) (width 1) (layer F.Cu) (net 3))
 (segment (start 172.72 90.17) (end 177.8 95.25) (width 1) (layer F.Cu) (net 3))
 (segment (start 172.72 81.28) (end 172.72 90.17) (width 1) (layer F.Cu) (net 3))
 (segment (start 171.877056 41.91) (end 170.18 41.91) (width 1) (layer F.Cu) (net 3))
 (segment (start 183.30707 41.91) (end 171.877056 41.91) (width 1) (layer F.Cu) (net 3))
 (segment (start 187.20999 66.79001) (end 187.20999 45.81292) (width 1) (layer F.Cu) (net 3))
 (segment (start 187.20999 45.81292) (end 183.30707 41.91) (width 1) (layer F.Cu) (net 3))
 (segment (start 172.72 81.28) (end 187.20999 66.79001) (width 1) (layer F.Cu) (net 3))
 (segment (start 144.78 63.25) (end 144.53 63.5) (width 1) (layer F.Cu) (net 4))
 (segment (start 144.78 54.61) (end 144.78 63.25) (width 1) (layer F.Cu) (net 4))
 (segment (start 144.78 49.53) (end 144.78 54.61) (width 1) (layer F.Cu) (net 4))
 (segment (start 153.67 45.72) (end 148.59 45.72) (width 1) (layer F.Cu) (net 4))
 (segment (start 148.59 45.72) (end 144.78 49.53) (width 1) (layer F.Cu) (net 4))
 (segment (start 173.99 111.76) (end 173.99 116.84) (width 1) (layer F.Cu) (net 9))
 (segment (start 173.99 116.84) (end 176.53 119.38) (width 1) (layer F.Cu) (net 9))
 (segment (start 176.53 119.38) (end 176.53 121.92) (width 1) (layer F.Cu) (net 9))
 (segment (start 147.32 63.75) (end 147.07 63.5) (width 1) (layer F.Cu) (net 13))
 (segment (start 147.32 77.47) (end 147.32 63.75) (width 1) (layer F.Cu) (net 13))
 (segment (start 171.45 111.76) (end 171.45 121.92) (width 1) (layer F.Cu) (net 10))
 (segment (start 149.86 63.75) (end 149.61 63.5) (width 1) (layer F.Cu) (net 14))
 (segment (start 149.86 77.47) (end 149.86 63.75) (width 1) (layer F.Cu) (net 14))
 (segment (start 168.91 100.33) (end 168.91 111.76) (width 1) (layer F.Cu) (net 11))
 (segment (start 152.15 65.79) (end 152.15 63.5) (width 1) (layer F.Cu) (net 20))
 (segment (start 153.67 77.47) (end 153.67 67.31) (width 1) (layer F.Cu) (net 20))
 (segment (start 153.67 67.31) (end 152.15 65.79) (width 1) (layer F.Cu) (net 20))
 (segment (start 166.37 111.76) (end 166.37 118.11) (width 1) (layer F.Cu) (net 8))
 (segment (start 143.51 118.15) (end 149.82 118.15) (width 1) (layer F.Cu) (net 8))
 (segment (start 149.82 118.15) (end 149.82 118.15) (width 1) (layer F.Cu) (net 8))
 (via (at 149.82 118.15) (size 2) (drill 1) (layers F.Cu B.Cu) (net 8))
 (segment (start 166.37 118.11) (end 163.83 115.57) (width 1) (layer F.Cu) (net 8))
 (segment (start 163.83 115.57) (end 162.56 115.57) (width 1) (layer F.Cu) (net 8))
 (segment (start 162.56 115.57) (end 162.56 115.57) (width 1) (layer F.Cu) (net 8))
 (via (at 162.56 115.57) (size 2) (drill 1) (layers F.Cu B.Cu) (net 8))
 (segment (start 152.4 115.57) (end 149.82 118.15) (width 1) (layer B.Cu) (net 8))
 (segment (start 162.56 115.57) (end 152.4 115.57) (width 1) (layer B.Cu) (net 8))
 (segment (start 154.69 65.79) (end 154.69 63.5) (width 1) (layer F.Cu) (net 21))
 (segment (start 156.21 77.47) (end 156.21 67.31) (width 1) (layer F.Cu) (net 21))
 (segment (start 156.21 67.31) (end 154.69 65.79) (width 1) (layer F.Cu) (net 21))
 (segment (start 181.61 102.83) (end 177.76 106.68) (width 1) (layer F.Cu) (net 12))
 (segment (start 181.61 100.33) (end 181.61 102.83) (width 1) (layer F.Cu) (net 12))
 (segment (start 177.76 106.68) (end 175.26 106.68) (width 1) (layer F.Cu) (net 12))
 (segment (start 161.29 111.76) (end 161.29 107.95) (width 1) (layer F.Cu) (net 12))
 (segment (start 161.29 107.95) (end 162.56 106.68) (width 1) (layer F.Cu) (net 12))
 (segment (start 162.56 106.68) (end 163.83 106.68) (width 1) (layer F.Cu) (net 12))
 (segment (start 163.83 106.68) (end 163.83 106.68) (width 1) (layer F.Cu) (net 12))
 (via (at 163.83 106.68) (size 2) (drill 1) (layers F.Cu B.Cu) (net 12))
 (segment (start 175.26 106.68) (end 175.26 106.68) (width 1) (layer F.Cu) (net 12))
 (via (at 175.26 106.68) (size 2) (drill 1) (layers F.Cu B.Cu) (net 12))
 (segment (start 163.83 106.68) (end 175.26 106.68) (width 1) (layer B.Cu) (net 12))
 (segment (start 157.23 65.79) (end 157.23 63.5) (width 1) (layer F.Cu) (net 22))
 (segment (start 158.75 77.47) (end 158.75 67.31) (width 1) (layer F.Cu) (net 22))
 (segment (start 158.75 67.31) (end 157.23 65.79) (width 1) (layer F.Cu) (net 22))
 (segment (start 129.54 76.2) (end 130.81 76.2) (width 1) (layer F.Cu) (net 23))
 (segment (start 130.81 76.2) (end 134.62 72.39) (width 1) (layer F.Cu) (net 23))
 (segment (start 134.62 72.39) (end 134.62 72.39) (width 1) (layer F.Cu) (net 23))
 (via (at 134.62 72.39) (size 2) (drill 1) (layers F.Cu B.Cu) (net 23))
 (segment (start 161.29 63.5) (end 161.29 72.39) (width 1) (layer F.Cu) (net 23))
 (segment (start 161.29 72.39) (end 161.29 72.39) (width 1) (layer F.Cu) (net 23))
 (via (at 161.29 72.39) (size 2) (drill 1) (layers F.Cu B.Cu) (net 23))
 (segment (start 134.62 72.39) (end 161.29 72.39) (width 1) (layer B.Cu) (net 23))
 (segment (start 162.56 54.61) (end 162.56 57.15) (width 1) (layer F.Cu) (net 5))
 (segment (start 162.56 57.15) (end 163.83 58.42) (width 1) (layer F.Cu) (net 5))
 (segment (start 163.83 58.42) (end 163.83 63.5) (width 1) (layer F.Cu) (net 5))
 (segment (start 156.17 54.61) (end 162.56 54.61) (width 1) (layer F.Cu) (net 5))
 (via (at 184.15 62.23) (size 2) (drill 1) (layers F.Cu B.Cu) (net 1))
 (via (at 181.61 90.17) (size 2) (drill 1) (layers F.Cu B.Cu) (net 1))
 (segment (start 144.78 77.47) (end 144.78 78.74) (width 1) (layer F.Cu) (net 1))
 (segment (start 144.78 78.74) (end 142.24 81.28) (width 1) (layer F.Cu) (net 1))
 (segment (start 142.24 81.28) (end 139.7 81.28) (width 1) (layer F.Cu) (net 1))
 (segment (start 139.7 81.28) (end 139.7 91.44) (width 1) (layer F.Cu) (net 1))
 (segment (start 129.54 81.28) (end 139.7 81.28) (width 1) (layer F.Cu) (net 1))
 (segment (start 139.7 95.25) (end 137.16 97.79) (width 1) (layer F.Cu) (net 1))
 (segment (start 139.7 91.44) (end 139.7 95.25) (width 1) (layer F.Cu) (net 1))
 (segment (start 171.45 126.92) (end 176.53 126.92) (width 1) (layer F.Cu) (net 1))
 (segment (start 163.83 133.35) (end 171.45 133.35) (width 1) (layer F.Cu) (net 1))
 (segment (start 153.67 111.76) (end 153.67 123.19) (width 1) (layer F.Cu) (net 1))
 (segment (start 171.45 133.35) (end 171.45 126.92) (width 1) (layer F.Cu) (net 1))
 (segment (start 153.67 123.19) (end 163.83 133.35) (width 1) (layer F.Cu) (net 1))
 (segment (start 153.67 111.76) (end 153.67 102.87) (width 1) (layer F.Cu) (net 1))
 (segment (start 153.67 102.87) (end 161.29 95.25) (width 1) (layer F.Cu) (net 1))
 (segment (start 161.37 95.33) (end 168.91 95.33) (width 1) (layer F.Cu) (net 1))
 (segment (start 161.29 95.25) (end 161.37 95.33) (width 1) (layer F.Cu) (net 1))
 (segment (start 140.24 102.87) (end 137.16 99.79) (width 1) (layer F.Cu) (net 1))
 (segment (start 137.16 99.79) (end 137.16 97.79) (width 1) (layer F.Cu) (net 1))
 (segment (start 153.67 102.87) (end 140.24 102.87) (width 1) (layer F.Cu) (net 1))
 (segment (start 156.17 45.72) (end 156.17 48.3) (width 1) (layer F.Cu) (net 1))
 (segment (start 153.67 50.8) (end 153.67 54.61) (width 1) (layer F.Cu) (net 1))
 (segment (start 156.17 48.3) (end 153.67 50.8) (width 1) (layer F.Cu) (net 1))
 (segment (start 180.34 57.15) (end 184.15 57.15) (width 1) (layer F.Cu) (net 1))
 (segment (start 184.15 57.15) (end 185.42 55.88) (width 1) (layer F.Cu) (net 1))
 (segment (start 185.42 55.88) (end 185.42 45.72) (width 1) (layer F.Cu) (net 1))
 (segment (start 185.42 45.72) (end 156.17 45.72) (width 1) (layer F.Cu) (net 1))
 (segment (start 151.13 120.65) (end 153.67 123.19) (width 1) (layer F.Cu) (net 1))
 (segment (start 143.51 120.65) (end 151.13 120.65) (width 1) (layer F.Cu) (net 1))
 (segment (start 166.37 72.39) (end 166.37 76.2) (width 1) (layer F.Cu) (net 1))
 (segment (start 166.37 76.2) (end 166.37 77.47) (width 1) (layer F.Cu) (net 1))
 (segment (start 166.37 77.47) (end 166.37 77.47) (width 1) (layer F.Cu) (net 1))
 (via (at 166.37 77.47) (size 2) (drill 1) (layers F.Cu B.Cu) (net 1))
 (segment (start 168.91 93.48) (end 166.37 90.94) (width 1) (layer F.Cu) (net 1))
 (segment (start 168.91 95.33) (end 168.91 93.48) (width 1) (layer F.Cu) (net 1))
 (segment (start 166.37 90.94) (end 166.37 87.63) (width 1) (layer F.Cu) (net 1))
 (segment (start 166.37 87.63) (end 166.37 87.63) (width 1) (layer F.Cu) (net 1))
 (via (at 166.37 87.63) (size 2) (drill 1) (layers F.Cu B.Cu) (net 1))
 (segment (start 166.37 77.47) (end 166.37 87.63) (width 1) (layer B.Cu) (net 1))
 (segment (start 139.7 91.44) (end 153.67 91.44) (width 1) (layer F.Cu) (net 1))
 (segment (start 153.67 91.44) (end 154.94 90.17) (width 1) (layer F.Cu) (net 1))
 (segment (start 154.94 90.17) (end 154.94 90.17) (width 1) (layer F.Cu) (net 1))
 (via (at 154.94 90.17) (size 2) (drill 1) (layers F.Cu B.Cu) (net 1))
 (segment (start 181.61 90.17) (end 154.94 90.17) (width 1) (layer B.Cu) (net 1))
 (segment (start 181.61 90.17) (end 185.42 86.36) (width 1) (layer F.Cu) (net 1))
 (segment (start 185.42 86.36) (end 185.42 76.2) (width 1) (layer F.Cu) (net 1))
 (segment (start 185.42 76.2) (end 185.42 76.2) (width 1) (layer F.Cu) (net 1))
 (via (at 185.42 76.2) (size 2) (drill 1) (layers F.Cu B.Cu) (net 1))
 (segment (start 184.15 57.15) (end 184.15 62.23) (width 1) (layer F.Cu) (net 1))
 (segment (start 184.15 74.93) (end 185.42 76.2) (width 1) (layer B.Cu) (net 1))
 (segment (start 184.15 62.23) (end 184.15 74.93) (width 1) (layer B.Cu) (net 1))
 (segment (start 166.37 54.61) (end 166.37 63.5) (width 1) (layer F.Cu) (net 6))
 (segment (start 166.37 63.5) (end 166.37 69.89) (width 1) (layer F.Cu) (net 6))
 (segment (start 151.13 114.3) (end 151.13 111.76) (width 1) (layer F.Cu) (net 17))
 (segment (start 116.84 111.76) (end 119.38 114.3) (width 1) (layer F.Cu) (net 17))
 (segment (start 121.92 68.58) (end 116.84 68.58) (width 1) (layer F.Cu) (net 17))
 (segment (start 119.38 114.3) (end 151.13 114.3) (width 1) (layer F.Cu) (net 17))
 (segment (start 116.84 68.58) (end 116.84 111.76) (width 1) (layer F.Cu) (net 17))
 (segment (start 170.18 54.61) (end 170.18 57.15) (width 1) (layer F.Cu) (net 7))
 (segment (start 170.18 57.15) (end 168.91 58.42) (width 1) (layer F.Cu) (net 7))
 (segment (start 168.91 58.42) (end 168.91 63.5) (width 1) (layer F.Cu) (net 7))
 (segment (start 172.72 52.07) (end 170.18 54.61) (width 1) (layer F.Cu) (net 7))
 (segment (start 180.34 52.07) (end 172.72 52.07) (width 1) (layer F.Cu) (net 7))
 (segment (start 171.45 68.62) (end 172.72 69.89) (width 1) (layer F.Cu) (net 18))
 (segment (start 171.45 63.5) (end 171.45 68.62) (width 1) (layer F.Cu) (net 18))
 (segment (start 178.34 69.89) (end 180.34 69.89) (width 1) (layer F.Cu) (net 19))
 (segment (start 173.99 65.54) (end 178.34 69.89) (width 1) (layer F.Cu) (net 19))
 (segment (start 173.99 63.5) (end 173.99 65.54) (width 1) (layer F.Cu) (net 19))
 (segment (start 136.91 65.79) (end 136.91 63.5) (width 1) (layer F.Cu) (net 16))
 (segment (start 121.92 66.04) (end 137.16 66.04) (width 1) (layer F.Cu) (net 16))
 (segment (start 137.16 66.04) (end 136.91 65.79) (width 1) (layer F.Cu) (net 16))
 (segment (start 121.92 63.5) (end 134.37 63.5) (width 1) (layer F.Cu) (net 15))
 (segment (start 134.5 78.74) (end 134.7 78.94) (width 1) (layer F.Cu) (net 2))
 (segment (start 129.54 78.74) (end 134.5 78.74) (width 1) (layer F.Cu) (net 2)))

